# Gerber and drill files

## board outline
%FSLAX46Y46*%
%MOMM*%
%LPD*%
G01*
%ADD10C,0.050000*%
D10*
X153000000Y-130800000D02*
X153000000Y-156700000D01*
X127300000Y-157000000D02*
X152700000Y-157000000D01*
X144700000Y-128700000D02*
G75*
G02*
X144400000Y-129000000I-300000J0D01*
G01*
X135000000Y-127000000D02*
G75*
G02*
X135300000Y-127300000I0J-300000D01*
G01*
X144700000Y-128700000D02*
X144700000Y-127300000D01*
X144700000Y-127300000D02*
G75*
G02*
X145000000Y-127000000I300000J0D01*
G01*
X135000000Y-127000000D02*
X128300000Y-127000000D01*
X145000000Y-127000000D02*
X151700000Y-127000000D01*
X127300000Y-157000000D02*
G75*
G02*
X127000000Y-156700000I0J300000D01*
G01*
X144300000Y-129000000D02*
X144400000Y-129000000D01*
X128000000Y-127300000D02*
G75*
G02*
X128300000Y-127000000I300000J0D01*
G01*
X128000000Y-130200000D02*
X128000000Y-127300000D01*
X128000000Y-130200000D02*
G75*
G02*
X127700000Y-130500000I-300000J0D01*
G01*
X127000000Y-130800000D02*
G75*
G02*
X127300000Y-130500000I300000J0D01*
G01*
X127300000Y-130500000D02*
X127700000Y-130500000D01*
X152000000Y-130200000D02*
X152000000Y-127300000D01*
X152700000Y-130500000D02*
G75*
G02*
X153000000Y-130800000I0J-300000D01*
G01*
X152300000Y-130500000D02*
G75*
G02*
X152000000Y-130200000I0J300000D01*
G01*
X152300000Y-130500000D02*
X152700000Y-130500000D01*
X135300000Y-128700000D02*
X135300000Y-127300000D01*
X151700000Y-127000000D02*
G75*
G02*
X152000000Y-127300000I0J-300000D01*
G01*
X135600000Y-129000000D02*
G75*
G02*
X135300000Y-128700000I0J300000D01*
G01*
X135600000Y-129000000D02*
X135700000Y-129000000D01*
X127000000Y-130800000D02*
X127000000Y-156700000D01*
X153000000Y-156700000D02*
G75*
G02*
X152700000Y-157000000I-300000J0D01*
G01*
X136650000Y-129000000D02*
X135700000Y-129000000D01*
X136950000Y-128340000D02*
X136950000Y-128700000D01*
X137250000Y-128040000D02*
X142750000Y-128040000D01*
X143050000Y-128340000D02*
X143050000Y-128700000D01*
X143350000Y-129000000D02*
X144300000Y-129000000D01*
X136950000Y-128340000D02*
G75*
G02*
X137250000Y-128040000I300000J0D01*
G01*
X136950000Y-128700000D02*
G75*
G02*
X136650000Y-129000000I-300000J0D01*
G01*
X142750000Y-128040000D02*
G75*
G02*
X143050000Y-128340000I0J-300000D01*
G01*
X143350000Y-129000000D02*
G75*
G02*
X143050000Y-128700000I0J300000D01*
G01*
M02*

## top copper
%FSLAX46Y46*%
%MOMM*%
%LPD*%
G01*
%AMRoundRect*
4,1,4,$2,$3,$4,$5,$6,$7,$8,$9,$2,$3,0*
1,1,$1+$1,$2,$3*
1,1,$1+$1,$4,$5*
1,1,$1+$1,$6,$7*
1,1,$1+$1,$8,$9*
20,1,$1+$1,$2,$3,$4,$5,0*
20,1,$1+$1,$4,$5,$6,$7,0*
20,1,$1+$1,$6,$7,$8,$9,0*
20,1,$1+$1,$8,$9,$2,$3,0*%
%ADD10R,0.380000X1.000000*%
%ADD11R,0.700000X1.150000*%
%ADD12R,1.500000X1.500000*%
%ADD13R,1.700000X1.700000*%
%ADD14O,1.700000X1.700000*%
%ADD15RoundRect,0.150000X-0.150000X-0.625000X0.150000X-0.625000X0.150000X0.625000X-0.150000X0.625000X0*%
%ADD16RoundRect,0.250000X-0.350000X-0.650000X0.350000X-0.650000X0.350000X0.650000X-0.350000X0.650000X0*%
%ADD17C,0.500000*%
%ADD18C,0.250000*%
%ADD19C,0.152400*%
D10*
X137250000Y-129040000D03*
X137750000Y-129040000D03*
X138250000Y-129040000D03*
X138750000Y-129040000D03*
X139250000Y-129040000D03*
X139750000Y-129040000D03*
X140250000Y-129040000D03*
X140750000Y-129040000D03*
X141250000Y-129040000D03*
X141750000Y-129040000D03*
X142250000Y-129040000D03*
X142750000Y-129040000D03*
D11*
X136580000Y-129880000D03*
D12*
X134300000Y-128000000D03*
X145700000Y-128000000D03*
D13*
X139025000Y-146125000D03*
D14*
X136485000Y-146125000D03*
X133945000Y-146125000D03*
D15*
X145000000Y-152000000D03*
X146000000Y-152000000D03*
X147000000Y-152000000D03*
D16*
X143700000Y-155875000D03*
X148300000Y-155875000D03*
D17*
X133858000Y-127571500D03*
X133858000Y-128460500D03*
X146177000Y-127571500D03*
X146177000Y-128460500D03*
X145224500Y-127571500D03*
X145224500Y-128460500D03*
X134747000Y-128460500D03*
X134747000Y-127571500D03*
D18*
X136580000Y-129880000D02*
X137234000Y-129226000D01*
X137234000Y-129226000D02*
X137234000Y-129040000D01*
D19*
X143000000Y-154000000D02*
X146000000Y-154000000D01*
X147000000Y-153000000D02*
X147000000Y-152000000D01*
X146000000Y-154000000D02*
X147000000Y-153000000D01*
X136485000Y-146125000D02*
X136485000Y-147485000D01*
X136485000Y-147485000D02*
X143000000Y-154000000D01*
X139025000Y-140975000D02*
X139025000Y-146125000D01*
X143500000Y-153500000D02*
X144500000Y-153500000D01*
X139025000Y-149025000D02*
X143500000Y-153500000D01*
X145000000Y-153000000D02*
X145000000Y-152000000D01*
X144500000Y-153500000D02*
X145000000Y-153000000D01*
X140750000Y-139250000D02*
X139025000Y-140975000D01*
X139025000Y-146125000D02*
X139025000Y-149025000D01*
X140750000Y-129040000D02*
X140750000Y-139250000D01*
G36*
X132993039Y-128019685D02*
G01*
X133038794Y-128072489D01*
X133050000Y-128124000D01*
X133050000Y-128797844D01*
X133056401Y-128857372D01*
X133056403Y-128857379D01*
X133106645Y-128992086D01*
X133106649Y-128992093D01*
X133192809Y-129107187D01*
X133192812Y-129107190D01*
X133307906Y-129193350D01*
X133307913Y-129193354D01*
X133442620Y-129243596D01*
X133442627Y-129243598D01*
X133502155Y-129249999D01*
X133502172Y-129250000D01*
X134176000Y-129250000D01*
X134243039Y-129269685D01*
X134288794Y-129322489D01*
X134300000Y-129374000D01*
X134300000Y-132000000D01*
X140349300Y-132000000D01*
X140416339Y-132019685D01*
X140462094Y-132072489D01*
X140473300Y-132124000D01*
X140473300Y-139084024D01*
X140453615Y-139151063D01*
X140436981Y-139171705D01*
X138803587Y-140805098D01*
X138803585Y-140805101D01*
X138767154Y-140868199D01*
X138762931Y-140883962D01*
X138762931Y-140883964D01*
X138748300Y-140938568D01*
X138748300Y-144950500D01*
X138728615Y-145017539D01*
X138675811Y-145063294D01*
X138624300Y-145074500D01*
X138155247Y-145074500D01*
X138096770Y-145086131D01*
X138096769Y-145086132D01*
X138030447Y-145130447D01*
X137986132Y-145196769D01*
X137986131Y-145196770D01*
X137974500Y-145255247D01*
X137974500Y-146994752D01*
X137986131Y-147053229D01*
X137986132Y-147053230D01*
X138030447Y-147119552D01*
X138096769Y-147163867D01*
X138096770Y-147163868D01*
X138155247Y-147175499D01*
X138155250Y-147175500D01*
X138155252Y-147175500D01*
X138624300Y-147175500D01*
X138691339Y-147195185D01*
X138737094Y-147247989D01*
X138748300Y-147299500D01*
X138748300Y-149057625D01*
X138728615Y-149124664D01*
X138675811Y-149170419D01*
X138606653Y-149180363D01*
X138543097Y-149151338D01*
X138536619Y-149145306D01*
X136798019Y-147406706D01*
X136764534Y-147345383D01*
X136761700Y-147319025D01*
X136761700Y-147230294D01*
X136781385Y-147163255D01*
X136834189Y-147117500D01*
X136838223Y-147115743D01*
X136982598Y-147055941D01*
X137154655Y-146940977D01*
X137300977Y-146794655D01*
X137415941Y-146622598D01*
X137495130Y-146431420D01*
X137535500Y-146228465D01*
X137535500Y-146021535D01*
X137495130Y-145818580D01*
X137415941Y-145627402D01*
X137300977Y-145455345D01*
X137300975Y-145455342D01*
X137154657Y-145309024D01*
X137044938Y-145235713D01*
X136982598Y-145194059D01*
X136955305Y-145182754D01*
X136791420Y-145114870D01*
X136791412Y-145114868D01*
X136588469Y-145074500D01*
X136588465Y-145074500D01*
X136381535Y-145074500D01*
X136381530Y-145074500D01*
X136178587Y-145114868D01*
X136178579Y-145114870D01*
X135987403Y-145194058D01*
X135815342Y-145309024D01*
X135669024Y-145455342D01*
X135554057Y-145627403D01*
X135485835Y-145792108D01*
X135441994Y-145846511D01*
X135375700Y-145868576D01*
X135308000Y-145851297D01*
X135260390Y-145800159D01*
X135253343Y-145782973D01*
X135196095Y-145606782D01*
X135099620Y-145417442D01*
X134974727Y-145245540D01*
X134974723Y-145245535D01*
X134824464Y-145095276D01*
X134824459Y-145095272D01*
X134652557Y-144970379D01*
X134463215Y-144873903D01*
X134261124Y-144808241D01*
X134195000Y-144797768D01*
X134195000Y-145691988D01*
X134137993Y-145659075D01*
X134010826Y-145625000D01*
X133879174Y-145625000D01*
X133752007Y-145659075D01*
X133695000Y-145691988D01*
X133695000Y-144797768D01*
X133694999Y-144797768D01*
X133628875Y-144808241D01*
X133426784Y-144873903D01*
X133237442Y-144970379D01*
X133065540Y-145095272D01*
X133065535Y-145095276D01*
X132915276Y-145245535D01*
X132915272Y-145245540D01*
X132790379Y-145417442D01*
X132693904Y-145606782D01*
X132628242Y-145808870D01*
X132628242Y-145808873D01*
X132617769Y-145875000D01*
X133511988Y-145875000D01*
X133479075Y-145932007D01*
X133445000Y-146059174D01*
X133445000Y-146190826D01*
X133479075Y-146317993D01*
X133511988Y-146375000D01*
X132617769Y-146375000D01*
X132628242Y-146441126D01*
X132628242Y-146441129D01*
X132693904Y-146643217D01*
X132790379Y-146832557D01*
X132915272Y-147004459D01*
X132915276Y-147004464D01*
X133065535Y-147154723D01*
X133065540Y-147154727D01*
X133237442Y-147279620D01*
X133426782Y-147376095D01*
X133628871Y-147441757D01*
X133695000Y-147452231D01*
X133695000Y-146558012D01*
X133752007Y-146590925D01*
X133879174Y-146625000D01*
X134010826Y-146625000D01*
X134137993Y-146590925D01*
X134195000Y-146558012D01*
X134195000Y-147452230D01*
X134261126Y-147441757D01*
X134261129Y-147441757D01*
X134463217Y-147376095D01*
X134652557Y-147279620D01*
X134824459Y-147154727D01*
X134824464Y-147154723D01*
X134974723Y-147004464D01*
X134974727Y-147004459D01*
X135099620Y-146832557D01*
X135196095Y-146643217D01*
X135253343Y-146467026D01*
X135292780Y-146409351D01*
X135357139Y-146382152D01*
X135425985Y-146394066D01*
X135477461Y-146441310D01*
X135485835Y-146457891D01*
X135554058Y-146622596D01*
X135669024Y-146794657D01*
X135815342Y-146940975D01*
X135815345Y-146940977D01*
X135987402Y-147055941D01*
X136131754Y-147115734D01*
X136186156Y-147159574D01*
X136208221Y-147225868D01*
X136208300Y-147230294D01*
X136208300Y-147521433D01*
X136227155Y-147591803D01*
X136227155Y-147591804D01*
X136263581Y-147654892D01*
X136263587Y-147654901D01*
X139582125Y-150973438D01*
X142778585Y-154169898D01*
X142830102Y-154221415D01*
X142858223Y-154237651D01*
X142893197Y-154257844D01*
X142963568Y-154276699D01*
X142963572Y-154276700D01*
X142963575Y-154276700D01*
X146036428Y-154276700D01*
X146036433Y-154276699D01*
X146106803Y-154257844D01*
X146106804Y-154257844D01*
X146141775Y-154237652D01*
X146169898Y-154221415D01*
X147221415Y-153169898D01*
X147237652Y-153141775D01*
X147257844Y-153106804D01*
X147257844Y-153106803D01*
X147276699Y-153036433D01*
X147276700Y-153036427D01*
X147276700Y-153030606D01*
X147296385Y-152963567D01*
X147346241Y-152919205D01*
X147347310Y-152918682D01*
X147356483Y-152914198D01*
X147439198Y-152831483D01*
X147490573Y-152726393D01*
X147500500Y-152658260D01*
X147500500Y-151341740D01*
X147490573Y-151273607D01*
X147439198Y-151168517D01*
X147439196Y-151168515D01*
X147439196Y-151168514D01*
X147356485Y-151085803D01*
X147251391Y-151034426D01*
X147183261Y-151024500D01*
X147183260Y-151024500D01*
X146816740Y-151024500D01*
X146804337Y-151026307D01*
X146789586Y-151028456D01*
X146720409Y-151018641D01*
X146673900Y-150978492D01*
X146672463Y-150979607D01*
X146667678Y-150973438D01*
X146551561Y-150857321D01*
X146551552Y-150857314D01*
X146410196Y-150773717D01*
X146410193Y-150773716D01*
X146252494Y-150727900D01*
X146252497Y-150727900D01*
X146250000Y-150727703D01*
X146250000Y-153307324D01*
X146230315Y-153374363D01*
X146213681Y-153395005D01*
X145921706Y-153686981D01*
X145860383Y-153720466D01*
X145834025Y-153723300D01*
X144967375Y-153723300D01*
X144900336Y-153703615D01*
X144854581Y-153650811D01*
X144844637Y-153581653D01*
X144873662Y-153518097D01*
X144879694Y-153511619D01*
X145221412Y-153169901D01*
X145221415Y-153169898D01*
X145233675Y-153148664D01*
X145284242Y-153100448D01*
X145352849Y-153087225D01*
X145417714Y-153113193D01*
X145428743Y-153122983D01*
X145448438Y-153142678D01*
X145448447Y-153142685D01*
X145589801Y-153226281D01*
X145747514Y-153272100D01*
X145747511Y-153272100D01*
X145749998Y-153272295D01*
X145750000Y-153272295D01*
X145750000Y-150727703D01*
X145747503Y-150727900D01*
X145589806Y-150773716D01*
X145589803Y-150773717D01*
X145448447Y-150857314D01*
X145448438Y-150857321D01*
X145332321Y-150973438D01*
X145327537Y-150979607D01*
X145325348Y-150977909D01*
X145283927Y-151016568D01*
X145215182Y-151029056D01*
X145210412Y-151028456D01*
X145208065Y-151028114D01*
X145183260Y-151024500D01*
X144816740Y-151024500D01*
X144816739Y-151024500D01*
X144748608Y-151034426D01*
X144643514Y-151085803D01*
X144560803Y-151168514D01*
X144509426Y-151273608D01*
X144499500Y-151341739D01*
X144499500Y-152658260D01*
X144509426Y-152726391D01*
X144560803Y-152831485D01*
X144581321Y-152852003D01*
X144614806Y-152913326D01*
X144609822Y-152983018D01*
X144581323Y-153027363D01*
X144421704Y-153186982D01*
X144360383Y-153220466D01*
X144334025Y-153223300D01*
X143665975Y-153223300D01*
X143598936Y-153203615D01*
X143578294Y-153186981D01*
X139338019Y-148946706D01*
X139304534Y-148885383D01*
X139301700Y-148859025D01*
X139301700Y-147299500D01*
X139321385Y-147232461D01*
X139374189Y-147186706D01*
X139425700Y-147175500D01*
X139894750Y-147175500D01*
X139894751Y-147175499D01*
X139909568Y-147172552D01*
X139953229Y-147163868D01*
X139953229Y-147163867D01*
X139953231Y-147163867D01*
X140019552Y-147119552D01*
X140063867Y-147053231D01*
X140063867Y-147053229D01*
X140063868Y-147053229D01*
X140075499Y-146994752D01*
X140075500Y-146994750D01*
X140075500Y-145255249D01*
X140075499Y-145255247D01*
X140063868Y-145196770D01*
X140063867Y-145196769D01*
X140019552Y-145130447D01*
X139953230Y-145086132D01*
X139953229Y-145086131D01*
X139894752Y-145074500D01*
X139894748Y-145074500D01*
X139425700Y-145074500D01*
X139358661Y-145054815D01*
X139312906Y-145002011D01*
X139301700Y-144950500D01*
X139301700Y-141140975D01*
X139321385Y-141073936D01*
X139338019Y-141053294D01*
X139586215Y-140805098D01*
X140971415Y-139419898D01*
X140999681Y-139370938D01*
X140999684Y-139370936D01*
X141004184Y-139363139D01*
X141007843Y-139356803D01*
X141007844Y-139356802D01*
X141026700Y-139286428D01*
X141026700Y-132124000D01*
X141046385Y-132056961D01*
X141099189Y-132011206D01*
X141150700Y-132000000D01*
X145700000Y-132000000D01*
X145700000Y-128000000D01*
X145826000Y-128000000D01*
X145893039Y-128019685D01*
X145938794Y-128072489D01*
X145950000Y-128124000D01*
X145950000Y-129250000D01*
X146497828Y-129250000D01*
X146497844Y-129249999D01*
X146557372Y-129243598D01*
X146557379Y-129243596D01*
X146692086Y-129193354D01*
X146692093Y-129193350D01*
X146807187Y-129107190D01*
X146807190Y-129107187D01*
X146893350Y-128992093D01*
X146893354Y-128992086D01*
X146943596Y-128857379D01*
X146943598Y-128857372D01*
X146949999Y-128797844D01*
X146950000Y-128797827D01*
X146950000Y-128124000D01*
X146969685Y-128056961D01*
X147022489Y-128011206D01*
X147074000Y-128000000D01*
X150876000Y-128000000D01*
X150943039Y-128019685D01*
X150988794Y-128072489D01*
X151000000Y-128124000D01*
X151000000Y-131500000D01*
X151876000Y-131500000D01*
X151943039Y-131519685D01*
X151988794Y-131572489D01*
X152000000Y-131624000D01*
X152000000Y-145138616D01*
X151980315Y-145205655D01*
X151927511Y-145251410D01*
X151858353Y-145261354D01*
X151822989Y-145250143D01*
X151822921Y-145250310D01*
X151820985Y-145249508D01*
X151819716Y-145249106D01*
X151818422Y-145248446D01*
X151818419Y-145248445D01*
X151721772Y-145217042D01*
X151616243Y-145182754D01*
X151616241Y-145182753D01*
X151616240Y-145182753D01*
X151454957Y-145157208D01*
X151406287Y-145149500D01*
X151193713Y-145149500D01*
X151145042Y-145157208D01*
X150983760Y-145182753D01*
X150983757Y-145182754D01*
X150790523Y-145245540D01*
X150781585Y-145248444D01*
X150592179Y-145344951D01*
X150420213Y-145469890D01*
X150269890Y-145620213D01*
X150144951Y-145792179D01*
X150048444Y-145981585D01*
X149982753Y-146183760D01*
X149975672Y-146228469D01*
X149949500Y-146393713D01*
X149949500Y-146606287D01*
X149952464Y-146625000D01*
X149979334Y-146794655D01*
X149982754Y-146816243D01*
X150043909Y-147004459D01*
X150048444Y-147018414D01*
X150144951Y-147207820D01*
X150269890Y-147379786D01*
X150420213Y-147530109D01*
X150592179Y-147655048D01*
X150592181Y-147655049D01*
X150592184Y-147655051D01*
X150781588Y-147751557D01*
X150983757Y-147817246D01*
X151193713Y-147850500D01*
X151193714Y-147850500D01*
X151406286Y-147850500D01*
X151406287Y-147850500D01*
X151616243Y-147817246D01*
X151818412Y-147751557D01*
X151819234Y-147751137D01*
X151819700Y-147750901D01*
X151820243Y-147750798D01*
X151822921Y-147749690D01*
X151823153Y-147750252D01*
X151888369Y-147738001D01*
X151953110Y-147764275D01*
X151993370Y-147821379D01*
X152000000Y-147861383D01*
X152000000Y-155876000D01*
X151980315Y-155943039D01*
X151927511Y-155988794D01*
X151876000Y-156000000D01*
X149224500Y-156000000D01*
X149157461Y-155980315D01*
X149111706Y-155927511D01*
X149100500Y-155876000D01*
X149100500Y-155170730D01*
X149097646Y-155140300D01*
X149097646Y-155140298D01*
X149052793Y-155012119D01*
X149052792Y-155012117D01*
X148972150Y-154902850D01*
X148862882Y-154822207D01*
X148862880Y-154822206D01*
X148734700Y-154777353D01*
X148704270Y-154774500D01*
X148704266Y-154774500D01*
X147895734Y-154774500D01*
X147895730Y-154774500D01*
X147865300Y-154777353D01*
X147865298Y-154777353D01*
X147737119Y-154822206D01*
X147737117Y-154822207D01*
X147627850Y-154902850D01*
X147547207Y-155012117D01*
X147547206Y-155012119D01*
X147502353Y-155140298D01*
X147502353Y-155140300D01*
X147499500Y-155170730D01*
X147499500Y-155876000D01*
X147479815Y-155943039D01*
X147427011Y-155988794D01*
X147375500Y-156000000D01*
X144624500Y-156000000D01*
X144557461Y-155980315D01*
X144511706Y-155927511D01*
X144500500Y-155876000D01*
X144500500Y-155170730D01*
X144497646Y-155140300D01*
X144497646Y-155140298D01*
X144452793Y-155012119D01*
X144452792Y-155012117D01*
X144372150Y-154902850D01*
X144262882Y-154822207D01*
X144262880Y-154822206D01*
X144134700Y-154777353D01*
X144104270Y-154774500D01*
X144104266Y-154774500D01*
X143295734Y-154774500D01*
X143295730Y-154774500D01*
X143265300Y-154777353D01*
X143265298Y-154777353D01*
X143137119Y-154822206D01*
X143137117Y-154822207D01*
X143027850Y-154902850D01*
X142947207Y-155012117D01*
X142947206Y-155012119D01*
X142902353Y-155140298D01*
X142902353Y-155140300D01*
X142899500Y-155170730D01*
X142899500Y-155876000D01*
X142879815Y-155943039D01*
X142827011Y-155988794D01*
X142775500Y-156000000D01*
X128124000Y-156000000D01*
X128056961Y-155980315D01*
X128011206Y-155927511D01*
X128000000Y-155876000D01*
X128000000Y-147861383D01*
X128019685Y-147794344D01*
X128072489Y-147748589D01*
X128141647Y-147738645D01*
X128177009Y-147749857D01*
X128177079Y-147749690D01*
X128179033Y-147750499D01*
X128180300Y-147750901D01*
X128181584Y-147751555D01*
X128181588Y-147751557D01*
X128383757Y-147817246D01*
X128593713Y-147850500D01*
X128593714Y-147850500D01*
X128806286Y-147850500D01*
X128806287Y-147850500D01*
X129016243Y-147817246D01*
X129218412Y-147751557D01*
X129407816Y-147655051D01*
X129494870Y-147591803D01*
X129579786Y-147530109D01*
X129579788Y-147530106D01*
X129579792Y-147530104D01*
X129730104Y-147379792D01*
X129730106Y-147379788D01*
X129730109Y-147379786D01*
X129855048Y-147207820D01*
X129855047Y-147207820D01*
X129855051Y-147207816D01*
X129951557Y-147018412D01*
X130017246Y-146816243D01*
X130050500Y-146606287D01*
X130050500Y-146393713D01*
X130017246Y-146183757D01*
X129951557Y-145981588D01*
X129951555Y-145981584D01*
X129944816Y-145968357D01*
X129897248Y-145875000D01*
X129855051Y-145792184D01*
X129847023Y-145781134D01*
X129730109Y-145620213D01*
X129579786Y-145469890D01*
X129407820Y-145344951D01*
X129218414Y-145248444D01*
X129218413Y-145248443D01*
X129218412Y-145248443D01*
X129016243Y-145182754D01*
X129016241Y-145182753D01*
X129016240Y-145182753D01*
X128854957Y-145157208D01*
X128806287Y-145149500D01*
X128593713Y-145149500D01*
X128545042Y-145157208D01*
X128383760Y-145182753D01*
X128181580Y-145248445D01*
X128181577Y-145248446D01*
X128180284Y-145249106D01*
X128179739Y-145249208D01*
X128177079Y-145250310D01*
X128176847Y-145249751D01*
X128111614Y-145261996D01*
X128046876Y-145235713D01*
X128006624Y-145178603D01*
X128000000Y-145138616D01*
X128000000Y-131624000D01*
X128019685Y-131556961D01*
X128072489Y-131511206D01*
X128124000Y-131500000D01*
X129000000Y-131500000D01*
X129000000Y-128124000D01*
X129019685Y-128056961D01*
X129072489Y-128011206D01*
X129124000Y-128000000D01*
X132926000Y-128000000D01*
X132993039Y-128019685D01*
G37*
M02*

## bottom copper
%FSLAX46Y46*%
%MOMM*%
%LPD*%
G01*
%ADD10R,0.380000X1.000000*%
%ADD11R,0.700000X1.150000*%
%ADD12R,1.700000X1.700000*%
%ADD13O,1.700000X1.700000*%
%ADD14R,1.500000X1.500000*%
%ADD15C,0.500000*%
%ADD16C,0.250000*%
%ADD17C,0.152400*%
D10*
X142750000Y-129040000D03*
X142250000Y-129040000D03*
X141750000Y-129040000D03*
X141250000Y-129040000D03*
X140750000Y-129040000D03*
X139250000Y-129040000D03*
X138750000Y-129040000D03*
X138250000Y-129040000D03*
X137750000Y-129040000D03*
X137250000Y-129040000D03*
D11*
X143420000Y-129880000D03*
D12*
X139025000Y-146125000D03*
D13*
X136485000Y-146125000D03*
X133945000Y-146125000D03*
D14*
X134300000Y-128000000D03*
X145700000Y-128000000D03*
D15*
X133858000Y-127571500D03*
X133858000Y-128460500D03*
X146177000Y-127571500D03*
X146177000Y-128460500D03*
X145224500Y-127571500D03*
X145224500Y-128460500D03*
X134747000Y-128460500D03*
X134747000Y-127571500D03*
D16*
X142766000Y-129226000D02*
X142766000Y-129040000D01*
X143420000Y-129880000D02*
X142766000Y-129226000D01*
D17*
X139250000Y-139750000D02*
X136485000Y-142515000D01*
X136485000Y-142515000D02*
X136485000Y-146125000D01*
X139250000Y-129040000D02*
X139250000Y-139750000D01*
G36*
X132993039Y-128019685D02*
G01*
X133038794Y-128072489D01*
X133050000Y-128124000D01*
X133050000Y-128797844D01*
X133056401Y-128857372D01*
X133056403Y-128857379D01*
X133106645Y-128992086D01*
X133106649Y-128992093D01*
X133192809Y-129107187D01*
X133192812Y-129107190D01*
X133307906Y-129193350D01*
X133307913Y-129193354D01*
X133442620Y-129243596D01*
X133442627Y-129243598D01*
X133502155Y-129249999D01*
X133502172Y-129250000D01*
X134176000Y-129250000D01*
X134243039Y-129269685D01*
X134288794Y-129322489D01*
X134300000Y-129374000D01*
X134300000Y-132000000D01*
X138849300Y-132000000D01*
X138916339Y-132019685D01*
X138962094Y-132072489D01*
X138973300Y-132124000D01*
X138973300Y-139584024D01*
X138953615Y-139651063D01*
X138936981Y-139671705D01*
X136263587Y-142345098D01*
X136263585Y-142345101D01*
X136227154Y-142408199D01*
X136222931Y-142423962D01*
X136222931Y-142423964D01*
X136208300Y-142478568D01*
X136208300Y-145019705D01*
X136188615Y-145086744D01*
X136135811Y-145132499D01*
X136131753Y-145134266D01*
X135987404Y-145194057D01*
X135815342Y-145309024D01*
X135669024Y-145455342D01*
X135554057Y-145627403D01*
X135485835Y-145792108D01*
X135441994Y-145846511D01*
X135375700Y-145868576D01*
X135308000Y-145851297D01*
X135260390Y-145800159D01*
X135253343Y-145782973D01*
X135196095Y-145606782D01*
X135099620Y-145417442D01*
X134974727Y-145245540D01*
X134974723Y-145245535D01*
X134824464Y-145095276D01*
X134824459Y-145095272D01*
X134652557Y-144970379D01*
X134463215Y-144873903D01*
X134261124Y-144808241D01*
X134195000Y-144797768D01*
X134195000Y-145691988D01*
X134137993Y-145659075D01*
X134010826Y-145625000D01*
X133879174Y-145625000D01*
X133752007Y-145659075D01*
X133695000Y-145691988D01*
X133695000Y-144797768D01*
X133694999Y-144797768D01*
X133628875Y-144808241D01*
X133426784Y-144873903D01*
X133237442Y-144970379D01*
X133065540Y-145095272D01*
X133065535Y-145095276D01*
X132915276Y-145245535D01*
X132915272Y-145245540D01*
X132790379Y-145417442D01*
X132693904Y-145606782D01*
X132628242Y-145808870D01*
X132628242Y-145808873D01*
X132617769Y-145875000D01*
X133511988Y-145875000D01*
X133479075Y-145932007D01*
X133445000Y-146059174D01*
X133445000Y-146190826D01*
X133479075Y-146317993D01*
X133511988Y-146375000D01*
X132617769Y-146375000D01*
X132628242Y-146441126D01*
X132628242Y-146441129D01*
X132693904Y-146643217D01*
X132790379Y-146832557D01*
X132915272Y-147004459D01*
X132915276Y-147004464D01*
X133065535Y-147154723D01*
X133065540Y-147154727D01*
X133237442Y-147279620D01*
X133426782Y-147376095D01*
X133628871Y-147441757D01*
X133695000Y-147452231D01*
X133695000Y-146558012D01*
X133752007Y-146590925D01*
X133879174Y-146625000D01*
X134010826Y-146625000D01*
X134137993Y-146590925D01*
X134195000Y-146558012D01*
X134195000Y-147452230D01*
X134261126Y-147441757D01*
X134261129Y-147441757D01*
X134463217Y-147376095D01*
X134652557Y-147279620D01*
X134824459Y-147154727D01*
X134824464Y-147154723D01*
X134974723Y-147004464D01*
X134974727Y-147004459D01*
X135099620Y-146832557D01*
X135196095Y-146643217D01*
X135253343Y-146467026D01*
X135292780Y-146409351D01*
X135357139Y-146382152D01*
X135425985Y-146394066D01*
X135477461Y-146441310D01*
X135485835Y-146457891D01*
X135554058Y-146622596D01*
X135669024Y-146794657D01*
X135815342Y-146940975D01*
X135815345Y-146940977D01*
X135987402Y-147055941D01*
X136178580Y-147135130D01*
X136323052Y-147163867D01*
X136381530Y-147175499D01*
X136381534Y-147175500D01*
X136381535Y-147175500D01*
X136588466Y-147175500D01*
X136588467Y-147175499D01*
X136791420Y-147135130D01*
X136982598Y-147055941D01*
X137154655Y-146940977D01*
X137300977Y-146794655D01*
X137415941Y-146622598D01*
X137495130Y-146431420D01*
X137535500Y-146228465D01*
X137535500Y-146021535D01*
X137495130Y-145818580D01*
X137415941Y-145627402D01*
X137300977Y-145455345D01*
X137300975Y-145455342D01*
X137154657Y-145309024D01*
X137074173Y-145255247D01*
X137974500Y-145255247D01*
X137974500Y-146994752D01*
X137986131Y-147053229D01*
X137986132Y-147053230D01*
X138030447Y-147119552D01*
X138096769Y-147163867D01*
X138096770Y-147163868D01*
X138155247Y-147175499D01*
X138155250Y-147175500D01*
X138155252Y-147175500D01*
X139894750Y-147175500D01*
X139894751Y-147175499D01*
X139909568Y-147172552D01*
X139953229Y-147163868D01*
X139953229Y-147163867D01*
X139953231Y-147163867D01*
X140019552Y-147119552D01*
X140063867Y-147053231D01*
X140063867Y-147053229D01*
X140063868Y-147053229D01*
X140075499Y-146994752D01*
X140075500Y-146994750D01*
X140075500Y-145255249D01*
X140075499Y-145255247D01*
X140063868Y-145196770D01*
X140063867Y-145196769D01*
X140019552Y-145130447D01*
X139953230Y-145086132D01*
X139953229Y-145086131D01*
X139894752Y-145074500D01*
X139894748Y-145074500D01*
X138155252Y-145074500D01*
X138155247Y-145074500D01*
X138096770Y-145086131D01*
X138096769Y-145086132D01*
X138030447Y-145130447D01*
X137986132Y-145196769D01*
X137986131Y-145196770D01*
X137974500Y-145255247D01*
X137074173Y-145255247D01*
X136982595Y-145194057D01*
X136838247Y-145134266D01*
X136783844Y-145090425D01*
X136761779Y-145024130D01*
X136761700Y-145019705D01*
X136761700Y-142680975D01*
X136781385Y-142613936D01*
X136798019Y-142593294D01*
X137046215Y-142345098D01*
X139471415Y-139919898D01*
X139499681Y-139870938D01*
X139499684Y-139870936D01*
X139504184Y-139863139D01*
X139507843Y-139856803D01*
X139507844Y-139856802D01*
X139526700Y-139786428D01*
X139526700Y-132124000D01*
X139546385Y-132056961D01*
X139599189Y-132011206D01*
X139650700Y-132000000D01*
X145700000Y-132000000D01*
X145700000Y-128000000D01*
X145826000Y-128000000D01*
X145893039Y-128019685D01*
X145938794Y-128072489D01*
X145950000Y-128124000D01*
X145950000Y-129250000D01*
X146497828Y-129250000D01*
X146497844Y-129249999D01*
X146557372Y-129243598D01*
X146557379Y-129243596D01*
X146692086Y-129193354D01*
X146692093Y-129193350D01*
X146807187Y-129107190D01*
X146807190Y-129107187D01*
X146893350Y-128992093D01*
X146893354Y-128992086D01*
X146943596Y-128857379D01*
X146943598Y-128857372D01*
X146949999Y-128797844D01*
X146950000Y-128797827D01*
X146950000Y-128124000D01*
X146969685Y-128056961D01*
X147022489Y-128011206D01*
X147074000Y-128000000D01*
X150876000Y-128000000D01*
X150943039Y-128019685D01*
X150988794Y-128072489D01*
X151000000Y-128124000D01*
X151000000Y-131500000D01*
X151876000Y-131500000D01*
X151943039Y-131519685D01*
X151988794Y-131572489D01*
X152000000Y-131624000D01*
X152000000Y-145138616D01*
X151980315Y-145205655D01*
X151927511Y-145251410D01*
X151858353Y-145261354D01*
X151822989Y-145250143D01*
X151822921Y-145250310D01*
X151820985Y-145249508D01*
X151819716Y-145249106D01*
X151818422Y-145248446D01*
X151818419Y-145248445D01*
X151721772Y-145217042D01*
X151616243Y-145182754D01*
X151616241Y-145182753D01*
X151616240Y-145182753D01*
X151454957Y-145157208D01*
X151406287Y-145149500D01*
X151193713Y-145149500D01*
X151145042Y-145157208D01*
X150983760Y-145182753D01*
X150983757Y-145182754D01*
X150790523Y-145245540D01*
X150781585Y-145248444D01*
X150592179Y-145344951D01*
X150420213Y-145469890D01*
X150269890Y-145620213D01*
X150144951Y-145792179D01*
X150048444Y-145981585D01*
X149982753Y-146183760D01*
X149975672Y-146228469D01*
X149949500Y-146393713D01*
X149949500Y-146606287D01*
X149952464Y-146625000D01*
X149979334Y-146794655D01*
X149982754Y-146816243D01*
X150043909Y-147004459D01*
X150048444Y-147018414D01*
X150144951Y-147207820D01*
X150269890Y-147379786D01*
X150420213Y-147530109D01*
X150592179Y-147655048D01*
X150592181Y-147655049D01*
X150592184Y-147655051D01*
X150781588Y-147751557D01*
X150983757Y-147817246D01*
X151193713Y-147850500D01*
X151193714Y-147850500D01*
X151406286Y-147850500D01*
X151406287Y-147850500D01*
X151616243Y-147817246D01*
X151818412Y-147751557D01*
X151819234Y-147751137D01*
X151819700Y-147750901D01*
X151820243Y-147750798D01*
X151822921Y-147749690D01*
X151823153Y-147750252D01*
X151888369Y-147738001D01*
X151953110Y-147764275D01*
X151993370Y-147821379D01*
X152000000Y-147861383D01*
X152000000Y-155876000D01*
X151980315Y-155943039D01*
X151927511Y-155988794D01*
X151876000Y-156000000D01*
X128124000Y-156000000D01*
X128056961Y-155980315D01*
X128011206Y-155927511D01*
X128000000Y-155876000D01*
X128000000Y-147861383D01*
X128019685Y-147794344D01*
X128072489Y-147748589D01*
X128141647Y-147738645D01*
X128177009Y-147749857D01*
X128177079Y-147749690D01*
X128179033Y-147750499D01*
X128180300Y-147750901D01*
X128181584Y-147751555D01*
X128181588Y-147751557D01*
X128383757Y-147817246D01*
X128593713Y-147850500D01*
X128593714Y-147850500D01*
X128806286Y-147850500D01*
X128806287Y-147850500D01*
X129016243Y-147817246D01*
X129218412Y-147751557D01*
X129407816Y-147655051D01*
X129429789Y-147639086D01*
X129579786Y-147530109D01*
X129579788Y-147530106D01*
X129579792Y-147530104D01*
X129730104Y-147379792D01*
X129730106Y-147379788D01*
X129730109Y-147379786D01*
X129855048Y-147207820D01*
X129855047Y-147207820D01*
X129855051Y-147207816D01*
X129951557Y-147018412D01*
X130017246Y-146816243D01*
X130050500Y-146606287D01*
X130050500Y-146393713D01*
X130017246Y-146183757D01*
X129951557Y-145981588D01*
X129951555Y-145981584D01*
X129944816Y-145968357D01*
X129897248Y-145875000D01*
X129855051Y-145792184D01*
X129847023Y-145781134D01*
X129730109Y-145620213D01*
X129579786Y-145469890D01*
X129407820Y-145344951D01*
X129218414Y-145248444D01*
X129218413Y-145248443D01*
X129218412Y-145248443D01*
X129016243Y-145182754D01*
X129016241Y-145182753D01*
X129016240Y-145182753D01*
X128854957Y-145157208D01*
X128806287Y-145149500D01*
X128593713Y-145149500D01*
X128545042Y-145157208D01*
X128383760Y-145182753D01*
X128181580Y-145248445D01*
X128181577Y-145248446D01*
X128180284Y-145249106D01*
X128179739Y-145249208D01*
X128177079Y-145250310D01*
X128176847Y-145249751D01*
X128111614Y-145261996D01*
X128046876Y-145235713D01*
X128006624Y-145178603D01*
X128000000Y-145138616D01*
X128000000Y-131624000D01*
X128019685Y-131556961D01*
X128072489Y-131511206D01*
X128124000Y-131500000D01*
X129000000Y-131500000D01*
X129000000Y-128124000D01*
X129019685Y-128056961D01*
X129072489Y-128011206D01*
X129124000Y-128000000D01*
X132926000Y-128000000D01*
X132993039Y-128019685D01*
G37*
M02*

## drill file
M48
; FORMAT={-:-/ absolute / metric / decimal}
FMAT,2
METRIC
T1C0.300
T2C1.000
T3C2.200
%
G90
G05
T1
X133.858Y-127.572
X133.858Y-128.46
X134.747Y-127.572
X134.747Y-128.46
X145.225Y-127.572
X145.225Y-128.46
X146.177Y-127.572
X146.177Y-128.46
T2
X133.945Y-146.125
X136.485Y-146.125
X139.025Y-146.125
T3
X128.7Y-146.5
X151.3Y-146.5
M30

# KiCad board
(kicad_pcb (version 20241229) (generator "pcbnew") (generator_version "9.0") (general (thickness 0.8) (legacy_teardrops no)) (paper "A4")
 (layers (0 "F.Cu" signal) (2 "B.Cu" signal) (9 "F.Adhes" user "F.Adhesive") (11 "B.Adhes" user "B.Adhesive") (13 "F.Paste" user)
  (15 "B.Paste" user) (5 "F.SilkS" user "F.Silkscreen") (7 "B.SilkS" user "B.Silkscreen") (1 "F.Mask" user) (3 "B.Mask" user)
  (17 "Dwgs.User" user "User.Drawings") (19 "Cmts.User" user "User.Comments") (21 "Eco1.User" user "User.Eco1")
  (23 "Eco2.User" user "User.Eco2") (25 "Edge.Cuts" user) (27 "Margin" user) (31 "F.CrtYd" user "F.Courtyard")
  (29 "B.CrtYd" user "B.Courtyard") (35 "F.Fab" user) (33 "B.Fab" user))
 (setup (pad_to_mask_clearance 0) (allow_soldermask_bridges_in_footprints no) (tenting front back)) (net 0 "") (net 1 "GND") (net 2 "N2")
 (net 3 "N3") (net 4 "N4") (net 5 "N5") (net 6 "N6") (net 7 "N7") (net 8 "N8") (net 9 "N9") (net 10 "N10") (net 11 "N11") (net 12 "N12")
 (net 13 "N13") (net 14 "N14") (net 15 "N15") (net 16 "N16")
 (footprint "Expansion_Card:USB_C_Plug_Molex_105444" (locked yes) (layer "F.Cu") (at 140 129)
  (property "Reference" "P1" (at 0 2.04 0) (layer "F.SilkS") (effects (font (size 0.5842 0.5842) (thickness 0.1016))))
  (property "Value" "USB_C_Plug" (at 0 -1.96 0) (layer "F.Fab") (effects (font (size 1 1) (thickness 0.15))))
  (fp_line (start -3.35 0) (end -4.3 0) (stroke (width 0.05) (type solid)) (layer "Edge.Cuts"))
  (fp_line (start -3.05 -0.66) (end -3.05 -0.3) (stroke (width 0.05) (type solid)) (layer "Edge.Cuts"))
  (fp_line (start -2.75 -0.96) (end 2.75 -0.96) (stroke (width 0.05) (type solid)) (layer "Edge.Cuts"))
  (fp_line (start 3.05 -0.66) (end 3.05 -0.3) (stroke (width 0.05) (type solid)) (layer "Edge.Cuts"))
  (fp_line (start 3.35 0) (end 4.3 0) (stroke (width 0.05) (type solid)) (layer "Edge.Cuts"))
  (fp_arc (start -3.05 -0.66) (mid -2.962132 -0.872132) (end -2.75 -0.96) (stroke (width 0.05) (type solid)) (layer "Edge.Cuts"))
  (fp_arc (start -3.05 -0.3) (mid -3.137868 -0.087868) (end -3.35 0) (stroke (width 0.05) (type solid)) (layer "Edge.Cuts"))
  (fp_arc (start 2.75 -0.96) (mid 2.962132 -0.872132) (end 3.05 -0.66) (stroke (width 0.05) (type solid)) (layer "Edge.Cuts"))
  (fp_arc (start 3.35 0) (mid 3.137868 -0.087868) (end 3.05 -0.3) (stroke (width 0.05) (type solid)) (layer "Edge.Cuts"))
  (pad "A1" smd rect (at -2.75 0.04) (size 0.38 1) (layers "F.Cu" "F.Mask" "F.Paste") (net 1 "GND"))
  (pad "A2" smd rect (at -2.25 0.04) (size 0.38 1) (layers "F.Cu" "F.Mask" "F.Paste") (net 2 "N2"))
  (pad "A3" smd rect (at -1.75 0.04) (size 0.38 1) (layers "F.Cu" "F.Mask" "F.Paste") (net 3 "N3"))
  (pad "A4" smd rect (at -1.25 0.04) (size 0.38 1) (layers "F.Cu" "F.Mask" "F.Paste") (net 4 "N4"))
  (pad "A5" smd rect (at -0.75 0.04) (size 0.38 1) (layers "F.Cu" "F.Mask" "F.Paste") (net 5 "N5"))
  (pad "A6" smd rect (at -0.25 0.04) (size 0.38 1) (layers "F.Cu" "F.Mask" "F.Paste") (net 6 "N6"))
  (pad "A7" smd rect (at 0.25 0.04) (size 0.38 1) (layers "F.Cu" "F.Mask" "F.Paste") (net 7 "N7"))
  (pad "A8" smd rect (at 0.75 0.04) (size 0.38 1) (layers "F.Cu" "F.Mask" "F.Paste") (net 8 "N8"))
  (pad "A9" smd rect (at 1.25 0.04) (size 0.38 1) (layers "F.Cu" "F.Mask" "F.Paste") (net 4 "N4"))
  (pad "A10" smd rect (at 1.75 0.04) (size 0.38 1) (layers "F.Cu" "F.Mask" "F.Paste") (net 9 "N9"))
  (pad "A11" smd rect (at 2.25 0.04) (size 0.38 1) (layers "F.Cu" "F.Mask" "F.Paste") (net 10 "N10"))
  (pad "A12" smd rect (at 2.75 0.04) (size 0.38 1) (layers "F.Cu" "F.Mask" "F.Paste") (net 1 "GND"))
  (pad "B1" smd rect (at 2.75 0.04) (size 0.38 1) (layers "B.Cu" "B.Mask" "B.Paste") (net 1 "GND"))
  (pad "B2" smd rect (at 2.25 0.04) (size 0.38 1) (layers "B.Cu" "B.Mask" "B.Paste") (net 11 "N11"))
  (pad "B3" smd rect (at 1.75 0.04) (size 0.38 1) (layers "B.Cu" "B.Mask" "B.Paste") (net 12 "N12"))
  (pad "B4" smd rect (at 1.25 0.04) (size 0.38 1) (layers "B.Cu" "B.Mask" "B.Paste") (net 4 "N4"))
  (pad "B5" smd rect (at 0.75 0.04) (size 0.38 1) (layers "B.Cu" "B.Mask" "B.Paste") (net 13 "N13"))
  (pad "B8" smd rect (at -0.75 0.04) (size 0.38 1) (layers "B.Cu" "B.Mask" "B.Paste") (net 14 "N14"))
  (pad "B9" smd rect (at -1.25 0.04) (size 0.38 1) (layers "B.Cu" "B.Mask" "B.Paste") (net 4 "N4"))
  (pad "B10" smd rect (at -1.75 0.04) (size 0.38 1) (layers "B.Cu" "B.Mask" "B.Paste") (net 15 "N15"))
  (pad "B11" smd rect (at -2.25 0.04) (size 0.38 1) (layers "B.Cu" "B.Mask" "B.Paste") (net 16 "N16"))
  (pad "B12" smd rect (at -2.75 0.04) (size 0.38 1) (layers "B.Cu" "B.Mask" "B.Paste") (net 1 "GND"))
  (pad "S1" smd rect (at -3.42 0.88) (size 0.7 1.15) (layers "F.Cu" "F.Mask" "F.Paste") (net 1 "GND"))
  (pad "S1" smd rect (at 3.42 0.88) (size 0.7 1.15) (layers "B.Cu" "B.Mask" "B.Paste") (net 1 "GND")))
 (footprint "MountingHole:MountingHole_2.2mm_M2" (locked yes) (layer "F.Cu") (at 128.7 146.5)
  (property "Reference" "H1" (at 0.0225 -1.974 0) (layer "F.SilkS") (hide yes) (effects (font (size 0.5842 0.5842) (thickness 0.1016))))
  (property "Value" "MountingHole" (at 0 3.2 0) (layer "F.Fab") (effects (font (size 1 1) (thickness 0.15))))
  (pad "" np_thru_hole circle (at 0 0) (size 2.2 2.2) (drill 2.2) (layers "*.Cu" "*.Mask")))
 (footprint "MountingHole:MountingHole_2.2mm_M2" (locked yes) (layer "F.Cu") (at 151.3 146.5)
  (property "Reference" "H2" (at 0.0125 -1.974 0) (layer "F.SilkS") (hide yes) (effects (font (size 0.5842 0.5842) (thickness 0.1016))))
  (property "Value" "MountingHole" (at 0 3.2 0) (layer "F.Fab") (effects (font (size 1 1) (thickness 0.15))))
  (pad "" np_thru_hole circle (at 0 0) (size 2.2 2.2) (drill 2.2) (layers "*.Cu" "*.Mask")))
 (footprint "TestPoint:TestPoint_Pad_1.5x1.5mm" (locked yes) (layer "F.Cu") (at 134.3 128)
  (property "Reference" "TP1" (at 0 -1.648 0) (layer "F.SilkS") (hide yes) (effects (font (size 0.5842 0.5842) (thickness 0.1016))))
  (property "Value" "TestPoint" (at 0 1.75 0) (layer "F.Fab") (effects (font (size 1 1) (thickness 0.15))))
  (pad "1" smd rect (at 0 0) (size 1.5 1.5) (layers "F.Cu" "F.Mask") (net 1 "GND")))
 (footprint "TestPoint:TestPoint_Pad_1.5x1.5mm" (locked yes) (layer "F.Cu") (at 145.7 128)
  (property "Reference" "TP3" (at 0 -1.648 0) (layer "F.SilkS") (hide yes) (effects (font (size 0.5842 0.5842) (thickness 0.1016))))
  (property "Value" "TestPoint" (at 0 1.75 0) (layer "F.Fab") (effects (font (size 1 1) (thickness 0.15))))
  (pad "1" smd rect (at 0 0) (size 1.5 1.5) (layers "F.Cu" "F.Mask") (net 1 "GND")))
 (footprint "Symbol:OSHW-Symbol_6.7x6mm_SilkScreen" (layer "F.Cu") (at 146.5 136.5)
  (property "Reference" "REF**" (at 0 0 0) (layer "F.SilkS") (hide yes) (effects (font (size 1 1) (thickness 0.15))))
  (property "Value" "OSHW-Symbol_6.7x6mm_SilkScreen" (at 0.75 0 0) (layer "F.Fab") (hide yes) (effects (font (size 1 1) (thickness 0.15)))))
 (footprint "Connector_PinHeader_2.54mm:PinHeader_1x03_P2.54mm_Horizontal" (layer "F.Cu") (at 139.025 146.125 -90)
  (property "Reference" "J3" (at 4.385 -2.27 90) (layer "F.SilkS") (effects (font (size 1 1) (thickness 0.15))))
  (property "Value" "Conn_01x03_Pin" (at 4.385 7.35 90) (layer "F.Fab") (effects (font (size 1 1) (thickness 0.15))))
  (pad "1" thru_hole rect (at 0 0 270) (size 1.7 1.7) (drill 1) (layers "*.Cu" "*.Mask") (remove_unused_layers no) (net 8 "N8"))
  (pad "2" thru_hole oval (at 0 2.54 270) (size 1.7 1.7) (drill 1) (layers "*.Cu" "*.Mask") (remove_unused_layers no) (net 14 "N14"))
  (pad "3" thru_hole oval (at 0 5.08 270) (size 1.7 1.7) (drill 1) (layers "*.Cu" "*.Mask") (remove_unused_layers no) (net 1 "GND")))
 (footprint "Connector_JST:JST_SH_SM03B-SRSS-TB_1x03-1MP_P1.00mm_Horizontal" (layer "F.Cu") (at 146 154)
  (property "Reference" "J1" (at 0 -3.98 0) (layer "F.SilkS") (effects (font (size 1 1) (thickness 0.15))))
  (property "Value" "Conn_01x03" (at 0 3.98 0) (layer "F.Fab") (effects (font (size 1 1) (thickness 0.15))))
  (pad "1" smd roundrect (at -1 -2) (size 0.6 1.55) (layers "F.Cu" "F.Mask" "F.Paste") (roundrect_rratio 0.25) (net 8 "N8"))
  (pad "2" smd roundrect (at 0 -2) (size 0.6 1.55) (layers "F.Cu" "F.Mask" "F.Paste") (roundrect_rratio 0.25) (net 1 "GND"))
  (pad "3" smd roundrect (at 1 -2) (size 0.6 1.55) (layers "F.Cu" "F.Mask" "F.Paste") (roundrect_rratio 0.25) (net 14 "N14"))
  (pad "MP" smd roundrect (at -2.3 1.875) (size 1.2 1.8) (layers "F.Cu" "F.Mask" "F.Paste") (roundrect_rratio 0.208333))
  (pad "MP" smd roundrect (at 2.3 1.875) (size 1.2 1.8) (layers "F.Cu" "F.Mask" "F.Paste") (roundrect_rratio 0.208333)))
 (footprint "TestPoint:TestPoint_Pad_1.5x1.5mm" (layer "B.Cu") (at 134.3 128)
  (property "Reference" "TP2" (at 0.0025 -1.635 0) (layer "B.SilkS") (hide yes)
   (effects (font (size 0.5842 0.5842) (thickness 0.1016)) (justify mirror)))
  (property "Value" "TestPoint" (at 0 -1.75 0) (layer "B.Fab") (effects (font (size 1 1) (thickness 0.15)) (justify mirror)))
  (pad "1" smd rect (at 0 0) (size 1.5 1.5) (layers "B.Cu" "B.Mask") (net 1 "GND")))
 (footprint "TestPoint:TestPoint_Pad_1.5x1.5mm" (layer "B.Cu") (at 145.7 128)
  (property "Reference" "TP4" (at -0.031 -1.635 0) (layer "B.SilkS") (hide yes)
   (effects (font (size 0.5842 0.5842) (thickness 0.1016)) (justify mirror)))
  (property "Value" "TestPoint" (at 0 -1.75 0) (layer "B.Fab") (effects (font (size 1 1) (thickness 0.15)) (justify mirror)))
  (pad "1" smd rect (at 0 0) (size 1.5 1.5) (layers "B.Cu" "B.Mask") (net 1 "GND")))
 (gr_line (start 153 130.8) (end 153 156.7) (stroke (width 0.05) (type solid)) (layer "Edge.Cuts"))
 (gr_line (start 127.3 157) (end 152.7 157) (stroke (width 0.05) (type solid)) (layer "Edge.Cuts"))
 (gr_arc (start 144.7 128.7) (mid 144.612132 128.912132) (end 144.4 129) (stroke (width 0.05) (type solid)) (layer "Edge.Cuts"))
 (gr_arc (start 135 127) (mid 135.212132 127.087868) (end 135.3 127.3) (stroke (width 0.05) (type solid)) (layer "Edge.Cuts"))
 (gr_line (start 144.7 128.7) (end 144.7 127.3) (stroke (width 0.05) (type solid)) (layer "Edge.Cuts"))
 (gr_arc (start 144.7 127.3) (mid 144.787868 127.087868) (end 145 127) (stroke (width 0.05) (type solid)) (layer "Edge.Cuts"))
 (gr_line (start 135 127) (end 128.3 127) (stroke (width 0.05) (type solid)) (layer "Edge.Cuts"))
 (gr_line (start 145 127) (end 151.7 127) (stroke (width 0.05) (type solid)) (layer "Edge.Cuts"))
 (gr_arc (start 127.3 157) (mid 127.087868 156.912132) (end 127 156.7) (stroke (width 0.05) (type solid)) (layer "Edge.Cuts"))
 (gr_line (start 144.3 129) (end 144.4 129) (stroke (width 0.05) (type solid)) (layer "Edge.Cuts"))
 (gr_arc (start 128 127.3) (mid 128.087868 127.087868) (end 128.3 127) (stroke (width 0.05) (type solid)) (layer "Edge.Cuts"))
 (gr_line (start 128 130.2) (end 128 127.3) (stroke (width 0.05) (type solid)) (layer "Edge.Cuts"))
 (gr_arc (start 128 130.2) (mid 127.912132 130.412132) (end 127.7 130.5) (stroke (width 0.05) (type solid)) (layer "Edge.Cuts"))
 (gr_arc (start 127 130.8) (mid 127.087868 130.587868) (end 127.3 130.5) (stroke (width 0.05) (type solid)) (layer "Edge.Cuts"))
 (gr_line (start 127.3 130.5) (end 127.7 130.5) (stroke (width 0.05) (type solid)) (layer "Edge.Cuts"))
 (gr_line (start 152 130.2) (end 152 127.3) (stroke (width 0.05) (type solid)) (layer "Edge.Cuts"))
 (gr_arc (start 152.7 130.5) (mid 152.912132 130.587868) (end 153 130.8) (stroke (width 0.05) (type solid)) (layer "Edge.Cuts"))
 (gr_arc (start 152.3 130.5) (mid 152.087868 130.412132) (end 152 130.2) (stroke (width 0.05) (type solid)) (layer "Edge.Cuts"))
 (gr_line (start 152.3 130.5) (end 152.7 130.5) (stroke (width 0.05) (type solid)) (layer "Edge.Cuts"))
 (gr_line (start 135.3 128.7) (end 135.3 127.3) (stroke (width 0.05) (type solid)) (layer "Edge.Cuts"))
 (gr_arc (start 151.7 127) (mid 151.912132 127.087868) (end 152 127.3) (stroke (width 0.05) (type solid)) (layer "Edge.Cuts"))
 (gr_arc (start 135.6 129) (mid 135.387868 128.912132) (end 135.3 128.7) (stroke (width 0.05) (type solid)) (layer "Edge.Cuts"))
 (gr_line (start 135.6 129) (end 135.7 129) (stroke (width 0.05) (type solid)) (layer "Edge.Cuts"))
 (gr_line (start 127 130.8) (end 127 156.7) (stroke (width 0.05) (type solid)) (layer "Edge.Cuts"))
 (gr_arc (start 153 156.7) (mid 152.912132 156.912132) (end 152.7 157) (stroke (width 0.05) (type solid)) (layer "Edge.Cuts"))
 (segment (start 136.58 129.88) (end 137.234 129.226) (width 0.25) (layer "F.Cu") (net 1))
 (segment (start 137.234 129.226) (end 137.234 129.04) (width 0.25) (layer "F.Cu") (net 1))
 (via (at 133.858 127.5715) (size 0.5) (drill 0.3) (layers "F.Cu" "B.Cu") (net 1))
 (via (at 133.858 128.4605) (size 0.5) (drill 0.3) (layers "F.Cu" "B.Cu") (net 1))
 (via (at 146.177 127.5715) (size 0.5) (drill 0.3) (layers "F.Cu" "B.Cu") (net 1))
 (via (at 146.177 128.4605) (size 0.5) (drill 0.3) (layers "F.Cu" "B.Cu") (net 1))
 (via (at 145.2245 127.5715) (size 0.5) (drill 0.3) (layers "F.Cu" "B.Cu") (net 1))
 (via (at 145.2245 128.4605) (size 0.5) (drill 0.3) (layers "F.Cu" "B.Cu") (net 1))
 (via (at 134.747 128.4605) (size 0.5) (drill 0.3) (layers "F.Cu" "B.Cu") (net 1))
 (via (at 134.747 127.5715) (size 0.5) (drill 0.3) (layers "F.Cu" "B.Cu") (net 1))
 (segment (start 142.766 129.226) (end 142.766 129.04) (width 0.25) (layer "B.Cu") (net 1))
 (segment (start 143.42 129.88) (end 142.766 129.226) (width 0.25) (layer "B.Cu") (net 1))
 (segment (start 143 154) (end 146 154) (width 0.1524) (layer "F.Cu") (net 14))
 (segment (start 147 153) (end 147 152) (width 0.1524) (layer "F.Cu") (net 14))
 (segment (start 146 154) (end 147 153) (width 0.1524) (layer "F.Cu") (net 14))
 (segment (start 136.485 146.125) (end 136.485 147.485) (width 0.1524) (layer "F.Cu") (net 14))
 (segment (start 136.485 147.485) (end 143 154) (width 0.1524) (layer "F.Cu") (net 14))
 (segment (start 139.25 139.75) (end 136.485 142.515) (width 0.1524) (layer "B.Cu") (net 14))
 (segment (start 136.485 142.515) (end 136.485 146.125) (width 0.1524) (layer "B.Cu") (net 14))
 (segment (start 139.25 129.04) (end 139.25 139.75) (width 0.1524) (layer "B.Cu") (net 14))
 (segment (start 139.025 140.975) (end 139.025 146.125) (width 0.1524) (layer "F.Cu") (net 8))
 (segment (start 143.5 153.5) (end 144.5 153.5) (width 0.1524) (layer "F.Cu") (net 8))
 (segment (start 139.025 149.025) (end 143.5 153.5) (width 0.1524) (layer "F.Cu") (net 8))
 (segment (start 145 153) (end 145 152) (width 0.1524) (layer "F.Cu") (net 8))
 (segment (start 144.5 153.5) (end 145 153) (width 0.1524) (layer "F.Cu") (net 8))
 (segment (start 140.75 139.25) (end 139.025 140.975) (width 0.1524) (layer "F.Cu") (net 8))
 (segment (start 139.025 146.125) (end 139.025 149.025) (width 0.1524) (layer "F.Cu") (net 8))
 (segment (start 140.75 129.04) (end 140.75 139.25) (width 0.1524) (layer "F.Cu") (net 8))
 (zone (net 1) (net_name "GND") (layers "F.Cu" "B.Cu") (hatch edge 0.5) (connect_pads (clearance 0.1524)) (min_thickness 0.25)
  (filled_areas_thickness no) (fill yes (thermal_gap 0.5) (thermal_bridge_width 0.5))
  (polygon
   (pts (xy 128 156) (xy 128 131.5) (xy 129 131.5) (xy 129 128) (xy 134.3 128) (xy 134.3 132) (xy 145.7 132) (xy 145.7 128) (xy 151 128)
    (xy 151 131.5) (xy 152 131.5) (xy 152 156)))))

